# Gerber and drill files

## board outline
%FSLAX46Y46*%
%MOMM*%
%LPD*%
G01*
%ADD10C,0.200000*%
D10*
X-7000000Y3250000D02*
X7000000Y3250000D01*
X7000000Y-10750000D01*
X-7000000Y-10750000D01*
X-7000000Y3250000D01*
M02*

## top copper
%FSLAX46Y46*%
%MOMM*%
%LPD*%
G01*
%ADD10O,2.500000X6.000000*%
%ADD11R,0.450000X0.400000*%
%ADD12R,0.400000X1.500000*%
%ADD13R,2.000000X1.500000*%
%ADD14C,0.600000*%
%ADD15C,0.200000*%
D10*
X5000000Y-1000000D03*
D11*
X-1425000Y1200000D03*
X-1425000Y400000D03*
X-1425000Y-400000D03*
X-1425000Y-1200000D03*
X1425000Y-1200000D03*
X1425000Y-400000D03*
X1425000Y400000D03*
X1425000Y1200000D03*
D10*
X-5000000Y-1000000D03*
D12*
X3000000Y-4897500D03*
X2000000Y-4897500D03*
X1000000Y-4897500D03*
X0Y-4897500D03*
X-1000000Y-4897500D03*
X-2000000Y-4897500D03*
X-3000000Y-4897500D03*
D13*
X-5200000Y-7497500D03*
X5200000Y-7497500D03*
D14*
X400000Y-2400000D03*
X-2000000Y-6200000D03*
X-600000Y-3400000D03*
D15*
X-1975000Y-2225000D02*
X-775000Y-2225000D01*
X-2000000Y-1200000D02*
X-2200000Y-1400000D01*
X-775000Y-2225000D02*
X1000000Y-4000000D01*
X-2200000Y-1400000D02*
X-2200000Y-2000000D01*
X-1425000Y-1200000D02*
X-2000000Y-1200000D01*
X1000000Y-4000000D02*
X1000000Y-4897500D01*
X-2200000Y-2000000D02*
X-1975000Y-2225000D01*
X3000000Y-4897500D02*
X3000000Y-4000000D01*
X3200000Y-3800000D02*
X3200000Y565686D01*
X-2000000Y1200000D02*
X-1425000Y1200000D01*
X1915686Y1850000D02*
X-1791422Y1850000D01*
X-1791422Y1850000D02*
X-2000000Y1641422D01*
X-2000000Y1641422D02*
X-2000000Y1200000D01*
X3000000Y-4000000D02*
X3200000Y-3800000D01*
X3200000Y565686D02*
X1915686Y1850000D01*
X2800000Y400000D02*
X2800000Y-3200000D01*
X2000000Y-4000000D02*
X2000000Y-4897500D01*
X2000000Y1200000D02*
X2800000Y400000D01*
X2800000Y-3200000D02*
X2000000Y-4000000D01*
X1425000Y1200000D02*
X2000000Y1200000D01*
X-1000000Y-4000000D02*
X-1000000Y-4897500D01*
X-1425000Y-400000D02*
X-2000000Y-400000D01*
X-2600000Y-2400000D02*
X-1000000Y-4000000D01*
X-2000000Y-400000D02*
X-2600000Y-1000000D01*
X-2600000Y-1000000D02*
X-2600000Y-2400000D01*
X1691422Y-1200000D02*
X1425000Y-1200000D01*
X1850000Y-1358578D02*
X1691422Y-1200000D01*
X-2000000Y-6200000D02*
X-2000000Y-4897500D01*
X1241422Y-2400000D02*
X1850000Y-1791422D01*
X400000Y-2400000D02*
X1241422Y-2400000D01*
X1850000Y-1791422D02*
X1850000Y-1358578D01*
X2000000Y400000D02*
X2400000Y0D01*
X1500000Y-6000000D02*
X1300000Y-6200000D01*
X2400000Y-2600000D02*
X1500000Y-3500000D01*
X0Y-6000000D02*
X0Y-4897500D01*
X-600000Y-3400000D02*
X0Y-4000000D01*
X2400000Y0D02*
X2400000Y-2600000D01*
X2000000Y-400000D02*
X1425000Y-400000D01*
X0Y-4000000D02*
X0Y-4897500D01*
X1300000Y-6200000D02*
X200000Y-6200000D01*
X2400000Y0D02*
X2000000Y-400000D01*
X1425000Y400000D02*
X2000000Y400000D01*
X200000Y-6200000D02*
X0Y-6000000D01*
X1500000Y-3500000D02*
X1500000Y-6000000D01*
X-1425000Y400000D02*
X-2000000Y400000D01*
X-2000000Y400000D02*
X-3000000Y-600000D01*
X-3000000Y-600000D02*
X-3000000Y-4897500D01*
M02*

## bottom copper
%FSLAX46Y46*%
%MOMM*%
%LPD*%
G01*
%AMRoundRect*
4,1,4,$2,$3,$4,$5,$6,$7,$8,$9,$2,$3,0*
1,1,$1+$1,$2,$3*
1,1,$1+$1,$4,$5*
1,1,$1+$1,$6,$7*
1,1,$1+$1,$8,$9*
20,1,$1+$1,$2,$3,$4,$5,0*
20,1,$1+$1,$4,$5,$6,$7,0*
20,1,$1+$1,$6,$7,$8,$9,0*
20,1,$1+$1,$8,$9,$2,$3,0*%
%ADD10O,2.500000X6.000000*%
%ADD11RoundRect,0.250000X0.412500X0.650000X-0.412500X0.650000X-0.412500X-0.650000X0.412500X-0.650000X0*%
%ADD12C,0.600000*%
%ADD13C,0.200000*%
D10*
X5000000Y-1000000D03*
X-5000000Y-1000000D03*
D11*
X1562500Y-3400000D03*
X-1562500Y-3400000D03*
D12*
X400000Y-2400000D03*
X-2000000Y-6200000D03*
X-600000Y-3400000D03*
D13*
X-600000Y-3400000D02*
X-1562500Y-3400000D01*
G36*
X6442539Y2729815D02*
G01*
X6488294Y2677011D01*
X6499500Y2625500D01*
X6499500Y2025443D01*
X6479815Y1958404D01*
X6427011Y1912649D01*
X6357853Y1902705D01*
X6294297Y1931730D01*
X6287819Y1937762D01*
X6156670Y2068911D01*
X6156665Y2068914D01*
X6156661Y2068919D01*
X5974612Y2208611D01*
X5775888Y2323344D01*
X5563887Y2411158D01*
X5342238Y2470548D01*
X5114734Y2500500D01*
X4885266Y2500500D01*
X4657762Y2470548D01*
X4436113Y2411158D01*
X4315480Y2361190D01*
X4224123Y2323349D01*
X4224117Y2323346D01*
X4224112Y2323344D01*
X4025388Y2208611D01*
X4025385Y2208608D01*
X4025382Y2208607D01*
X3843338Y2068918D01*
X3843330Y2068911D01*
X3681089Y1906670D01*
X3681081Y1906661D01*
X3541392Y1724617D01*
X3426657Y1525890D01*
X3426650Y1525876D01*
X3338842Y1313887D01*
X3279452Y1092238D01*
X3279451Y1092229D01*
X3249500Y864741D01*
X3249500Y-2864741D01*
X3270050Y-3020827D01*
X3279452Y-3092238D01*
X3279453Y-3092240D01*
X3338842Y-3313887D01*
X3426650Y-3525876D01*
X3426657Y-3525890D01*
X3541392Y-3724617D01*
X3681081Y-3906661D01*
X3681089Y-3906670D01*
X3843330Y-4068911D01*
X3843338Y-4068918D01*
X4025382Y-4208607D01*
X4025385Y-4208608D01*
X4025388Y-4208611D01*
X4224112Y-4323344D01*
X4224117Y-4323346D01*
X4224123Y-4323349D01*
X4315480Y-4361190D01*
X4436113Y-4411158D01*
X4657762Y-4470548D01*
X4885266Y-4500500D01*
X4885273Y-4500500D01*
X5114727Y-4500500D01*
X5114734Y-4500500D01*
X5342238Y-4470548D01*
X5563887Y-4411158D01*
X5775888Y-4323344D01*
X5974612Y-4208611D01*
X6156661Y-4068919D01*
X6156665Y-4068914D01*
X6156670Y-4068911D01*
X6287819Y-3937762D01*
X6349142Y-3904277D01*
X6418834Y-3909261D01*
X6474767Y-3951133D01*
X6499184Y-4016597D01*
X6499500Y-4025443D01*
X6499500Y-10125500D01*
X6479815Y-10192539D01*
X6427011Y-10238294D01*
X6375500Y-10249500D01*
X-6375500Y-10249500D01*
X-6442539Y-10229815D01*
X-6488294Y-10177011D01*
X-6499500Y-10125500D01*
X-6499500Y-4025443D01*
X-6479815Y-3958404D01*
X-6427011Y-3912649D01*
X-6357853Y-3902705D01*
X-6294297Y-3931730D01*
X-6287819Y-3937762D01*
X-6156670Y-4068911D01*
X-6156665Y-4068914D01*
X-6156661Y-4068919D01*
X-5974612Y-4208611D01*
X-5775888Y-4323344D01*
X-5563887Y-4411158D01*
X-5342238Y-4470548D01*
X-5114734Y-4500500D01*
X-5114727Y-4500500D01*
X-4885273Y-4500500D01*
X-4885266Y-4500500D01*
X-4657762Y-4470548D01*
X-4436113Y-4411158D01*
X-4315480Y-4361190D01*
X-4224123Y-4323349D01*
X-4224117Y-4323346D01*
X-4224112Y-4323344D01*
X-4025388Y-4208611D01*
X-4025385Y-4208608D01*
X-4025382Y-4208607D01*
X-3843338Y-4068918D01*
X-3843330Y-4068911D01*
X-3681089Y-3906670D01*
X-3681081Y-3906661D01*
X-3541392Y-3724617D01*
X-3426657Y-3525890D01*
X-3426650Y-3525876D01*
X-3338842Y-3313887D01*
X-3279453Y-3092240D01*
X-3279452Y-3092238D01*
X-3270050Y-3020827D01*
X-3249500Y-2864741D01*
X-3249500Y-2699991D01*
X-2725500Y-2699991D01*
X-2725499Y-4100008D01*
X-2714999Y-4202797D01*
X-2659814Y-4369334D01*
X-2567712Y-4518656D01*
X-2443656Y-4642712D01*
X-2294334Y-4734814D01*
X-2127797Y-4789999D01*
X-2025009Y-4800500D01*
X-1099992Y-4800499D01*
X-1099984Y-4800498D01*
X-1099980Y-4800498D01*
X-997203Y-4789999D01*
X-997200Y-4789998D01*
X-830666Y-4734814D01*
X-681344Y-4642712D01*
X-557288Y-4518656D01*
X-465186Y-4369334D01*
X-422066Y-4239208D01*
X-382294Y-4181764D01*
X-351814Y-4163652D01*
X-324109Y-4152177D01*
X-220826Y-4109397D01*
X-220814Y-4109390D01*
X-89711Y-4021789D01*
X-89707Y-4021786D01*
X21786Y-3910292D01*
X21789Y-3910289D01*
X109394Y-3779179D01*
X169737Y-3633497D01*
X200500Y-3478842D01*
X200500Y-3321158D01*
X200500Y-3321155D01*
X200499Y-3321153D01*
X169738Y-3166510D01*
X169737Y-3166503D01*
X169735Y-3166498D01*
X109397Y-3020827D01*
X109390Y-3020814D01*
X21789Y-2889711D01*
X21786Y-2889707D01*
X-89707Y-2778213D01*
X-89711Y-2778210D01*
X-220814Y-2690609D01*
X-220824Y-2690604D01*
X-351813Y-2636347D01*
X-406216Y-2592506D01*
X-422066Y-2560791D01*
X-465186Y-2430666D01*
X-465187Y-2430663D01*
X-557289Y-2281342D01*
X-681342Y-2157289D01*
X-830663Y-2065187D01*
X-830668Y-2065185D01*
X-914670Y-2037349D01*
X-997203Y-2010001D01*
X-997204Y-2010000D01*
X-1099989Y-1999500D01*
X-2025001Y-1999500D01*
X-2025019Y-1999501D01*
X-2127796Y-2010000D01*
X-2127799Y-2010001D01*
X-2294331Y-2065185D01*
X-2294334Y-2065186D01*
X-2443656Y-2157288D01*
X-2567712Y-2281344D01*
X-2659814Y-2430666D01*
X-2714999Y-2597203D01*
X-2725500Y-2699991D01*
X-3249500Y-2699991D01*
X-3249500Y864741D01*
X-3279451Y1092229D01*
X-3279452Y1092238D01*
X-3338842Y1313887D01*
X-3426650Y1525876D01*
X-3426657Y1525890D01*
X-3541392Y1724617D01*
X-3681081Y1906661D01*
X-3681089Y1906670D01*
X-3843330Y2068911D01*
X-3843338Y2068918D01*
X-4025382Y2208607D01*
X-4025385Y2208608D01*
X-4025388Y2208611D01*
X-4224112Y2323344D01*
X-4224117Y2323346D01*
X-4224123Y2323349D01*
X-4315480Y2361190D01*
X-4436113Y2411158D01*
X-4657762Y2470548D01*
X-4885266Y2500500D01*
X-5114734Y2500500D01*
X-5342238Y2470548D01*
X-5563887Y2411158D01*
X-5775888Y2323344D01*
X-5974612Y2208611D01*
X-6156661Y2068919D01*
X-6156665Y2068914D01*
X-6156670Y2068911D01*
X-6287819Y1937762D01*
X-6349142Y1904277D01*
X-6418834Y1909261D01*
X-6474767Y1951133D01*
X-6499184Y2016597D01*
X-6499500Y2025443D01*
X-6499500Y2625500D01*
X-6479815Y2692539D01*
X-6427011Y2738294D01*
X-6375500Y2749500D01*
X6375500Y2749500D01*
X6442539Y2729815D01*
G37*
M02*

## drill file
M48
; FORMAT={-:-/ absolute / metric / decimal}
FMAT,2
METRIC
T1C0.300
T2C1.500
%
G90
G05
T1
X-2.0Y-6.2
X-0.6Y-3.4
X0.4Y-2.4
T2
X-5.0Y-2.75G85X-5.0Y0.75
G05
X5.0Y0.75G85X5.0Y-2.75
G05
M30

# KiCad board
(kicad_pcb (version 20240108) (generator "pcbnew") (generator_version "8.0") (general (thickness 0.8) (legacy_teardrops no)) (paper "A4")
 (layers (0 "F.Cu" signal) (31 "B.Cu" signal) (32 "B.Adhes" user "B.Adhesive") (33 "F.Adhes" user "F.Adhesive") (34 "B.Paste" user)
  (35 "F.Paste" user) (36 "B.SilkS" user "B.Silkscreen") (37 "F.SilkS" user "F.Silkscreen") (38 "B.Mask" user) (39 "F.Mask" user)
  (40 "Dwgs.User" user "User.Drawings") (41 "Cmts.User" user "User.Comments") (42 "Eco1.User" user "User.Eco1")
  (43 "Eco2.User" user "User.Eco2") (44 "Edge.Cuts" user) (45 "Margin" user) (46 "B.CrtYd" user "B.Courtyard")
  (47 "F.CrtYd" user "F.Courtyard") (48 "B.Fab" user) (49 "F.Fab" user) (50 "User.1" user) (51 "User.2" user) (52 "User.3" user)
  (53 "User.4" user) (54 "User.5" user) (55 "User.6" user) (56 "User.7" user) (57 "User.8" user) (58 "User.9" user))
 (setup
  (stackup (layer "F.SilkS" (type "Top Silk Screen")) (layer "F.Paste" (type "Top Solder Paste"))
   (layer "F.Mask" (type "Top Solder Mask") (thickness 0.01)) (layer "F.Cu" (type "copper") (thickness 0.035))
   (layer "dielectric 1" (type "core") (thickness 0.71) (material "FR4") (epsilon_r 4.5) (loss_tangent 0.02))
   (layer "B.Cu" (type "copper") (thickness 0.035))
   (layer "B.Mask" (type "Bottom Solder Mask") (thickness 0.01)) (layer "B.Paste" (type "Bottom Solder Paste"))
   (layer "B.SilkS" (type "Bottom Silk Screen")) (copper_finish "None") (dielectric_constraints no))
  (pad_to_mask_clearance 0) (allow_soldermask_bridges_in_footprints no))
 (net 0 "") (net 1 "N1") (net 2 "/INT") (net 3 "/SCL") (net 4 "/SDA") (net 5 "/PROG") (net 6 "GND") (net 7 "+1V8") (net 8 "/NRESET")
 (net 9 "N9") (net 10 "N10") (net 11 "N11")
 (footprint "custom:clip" (layer "F.Cu") (at 5 1 -90)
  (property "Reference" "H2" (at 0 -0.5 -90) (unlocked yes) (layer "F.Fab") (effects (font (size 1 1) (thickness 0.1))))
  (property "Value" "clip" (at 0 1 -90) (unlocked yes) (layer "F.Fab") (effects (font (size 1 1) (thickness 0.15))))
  (pad "1" thru_hole oval (at 0 0 270) (size 6 2.5) (drill oval 5 1.5) (layers "*.Cu" "*.Mask") (remove_unused_layers no) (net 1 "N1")
   (thermal_bridge_angle 45)))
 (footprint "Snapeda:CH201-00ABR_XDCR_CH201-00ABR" (layer "F.Cu") (at 0 0)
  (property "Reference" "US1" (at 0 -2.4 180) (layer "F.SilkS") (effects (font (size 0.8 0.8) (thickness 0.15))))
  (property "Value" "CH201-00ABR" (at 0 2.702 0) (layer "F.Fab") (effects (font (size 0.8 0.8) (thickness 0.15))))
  (pad "1" smd rect (at -1.425 -1.2) (size 0.45 0.4) (layers "F.Cu") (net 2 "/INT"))
  (pad "2" smd rect (at -1.425 -0.4) (size 0.45 0.4) (layers "F.Cu") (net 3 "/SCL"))
  (pad "3" smd rect (at -1.425 0.4) (size 0.45 0.4) (layers "F.Cu") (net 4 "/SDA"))
  (pad "4" smd rect (at -1.425 1.2) (size 0.45 0.4) (layers "F.Cu") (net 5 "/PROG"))
  (pad "5" smd rect (at 1.425 1.2) (size 0.45 0.4) (layers "F.Cu") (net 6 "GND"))
  (pad "6" smd rect (at 1.425 0.4) (size 0.45 0.4) (layers "F.Cu") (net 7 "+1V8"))
  (pad "7" smd rect (at 1.425 -0.4) (size 0.45 0.4) (layers "F.Cu") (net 7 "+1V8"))
  (pad "8" smd rect (at 1.425 -1.2) (size 0.45 0.4) (layers "F.Cu") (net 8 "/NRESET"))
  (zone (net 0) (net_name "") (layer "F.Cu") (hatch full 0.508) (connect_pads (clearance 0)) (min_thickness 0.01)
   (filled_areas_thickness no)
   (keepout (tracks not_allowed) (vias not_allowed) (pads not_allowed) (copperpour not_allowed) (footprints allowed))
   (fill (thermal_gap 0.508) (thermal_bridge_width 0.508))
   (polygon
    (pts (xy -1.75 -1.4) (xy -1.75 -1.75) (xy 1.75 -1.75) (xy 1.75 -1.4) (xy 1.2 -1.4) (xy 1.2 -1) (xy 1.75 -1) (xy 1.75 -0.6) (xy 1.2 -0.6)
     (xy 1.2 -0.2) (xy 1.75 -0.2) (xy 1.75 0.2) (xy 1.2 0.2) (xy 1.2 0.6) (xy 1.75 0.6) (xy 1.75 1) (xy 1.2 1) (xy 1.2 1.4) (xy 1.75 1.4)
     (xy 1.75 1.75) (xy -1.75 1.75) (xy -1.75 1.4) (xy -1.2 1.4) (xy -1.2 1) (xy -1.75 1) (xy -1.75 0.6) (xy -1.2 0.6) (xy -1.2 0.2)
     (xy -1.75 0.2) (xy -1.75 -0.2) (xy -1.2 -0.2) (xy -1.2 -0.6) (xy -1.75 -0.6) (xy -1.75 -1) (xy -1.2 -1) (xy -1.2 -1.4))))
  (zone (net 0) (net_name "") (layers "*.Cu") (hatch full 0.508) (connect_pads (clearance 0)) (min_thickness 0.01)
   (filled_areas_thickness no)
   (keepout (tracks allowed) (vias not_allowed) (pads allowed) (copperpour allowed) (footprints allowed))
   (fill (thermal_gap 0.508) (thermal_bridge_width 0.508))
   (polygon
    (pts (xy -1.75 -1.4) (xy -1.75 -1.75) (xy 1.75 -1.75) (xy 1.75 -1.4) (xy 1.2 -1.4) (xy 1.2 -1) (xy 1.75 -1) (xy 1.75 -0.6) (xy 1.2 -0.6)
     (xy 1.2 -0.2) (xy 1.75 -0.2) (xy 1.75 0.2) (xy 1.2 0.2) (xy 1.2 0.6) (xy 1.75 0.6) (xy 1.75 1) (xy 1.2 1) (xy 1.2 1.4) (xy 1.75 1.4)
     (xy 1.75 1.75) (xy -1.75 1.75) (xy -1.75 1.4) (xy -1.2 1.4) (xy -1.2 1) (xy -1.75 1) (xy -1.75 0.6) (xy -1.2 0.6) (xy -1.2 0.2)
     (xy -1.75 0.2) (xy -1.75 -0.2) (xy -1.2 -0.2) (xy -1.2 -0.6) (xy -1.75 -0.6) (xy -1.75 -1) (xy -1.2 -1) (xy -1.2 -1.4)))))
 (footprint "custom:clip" (layer "F.Cu") (at -5 1 90)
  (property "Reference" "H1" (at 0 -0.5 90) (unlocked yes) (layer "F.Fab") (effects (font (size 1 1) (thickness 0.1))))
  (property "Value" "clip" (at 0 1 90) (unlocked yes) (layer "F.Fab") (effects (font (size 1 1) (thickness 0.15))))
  (pad "1" thru_hole oval (at 0 0 90) (size 6 2.5) (drill oval 5 1.5) (layers "*.Cu" "*.Mask") (remove_unused_layers no) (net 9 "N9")
   (thermal_bridge_angle 45)))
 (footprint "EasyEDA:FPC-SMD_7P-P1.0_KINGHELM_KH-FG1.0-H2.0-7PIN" (layer "F.Cu") (at 0 6.1975)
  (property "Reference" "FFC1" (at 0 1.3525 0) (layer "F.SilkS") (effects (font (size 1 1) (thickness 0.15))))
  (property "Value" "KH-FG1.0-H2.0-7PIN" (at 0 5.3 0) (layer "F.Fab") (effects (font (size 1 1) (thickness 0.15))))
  (pad "1" smd rect (at 3 -1.3 180) (size 0.4 1.5) (layers "F.Cu" "F.Paste" "F.Mask") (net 2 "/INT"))
  (pad "2" smd rect (at 2 -1.3 180) (size 0.4 1.5) (layers "F.Cu" "F.Paste" "F.Mask") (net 8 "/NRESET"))
  (pad "3" smd rect (at 1 -1.3 180) (size 0.4 1.5) (layers "F.Cu" "F.Paste" "F.Mask") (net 5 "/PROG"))
  (pad "4" smd rect (at 0 -1.3 180) (size 0.4 1.5) (layers "F.Cu" "F.Paste" "F.Mask") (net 7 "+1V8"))
  (pad "5" smd rect (at -1 -1.3 180) (size 0.4 1.5) (layers "F.Cu" "F.Paste" "F.Mask") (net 4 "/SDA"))
  (pad "6" smd rect (at -2 -1.3 180) (size 0.4 1.5) (layers "F.Cu" "F.Paste" "F.Mask") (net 6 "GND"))
  (pad "7" smd rect (at -3 -1.3 180) (size 0.4 1.5) (layers "F.Cu" "F.Paste" "F.Mask") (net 3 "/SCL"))
  (pad "8" smd rect (at -5.2 1.3 180) (size 2 1.5) (layers "F.Cu" "F.Paste" "F.Mask") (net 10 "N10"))
  (pad "9" smd rect (at 5.2 1.3 180) (size 2 1.5) (layers "F.Cu" "F.Paste" "F.Mask") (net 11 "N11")))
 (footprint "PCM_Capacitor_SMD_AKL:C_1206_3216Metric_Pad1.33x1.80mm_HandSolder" (layer "B.Cu") (at 0 3.4 180)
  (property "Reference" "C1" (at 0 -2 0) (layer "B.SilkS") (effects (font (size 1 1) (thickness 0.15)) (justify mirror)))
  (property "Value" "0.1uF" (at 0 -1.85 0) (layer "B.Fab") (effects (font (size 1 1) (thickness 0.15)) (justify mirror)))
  (pad "1" smd roundrect (at -1.5625 0 180) (size 1.325 1.8) (layers "B.Cu" "B.Paste" "B.Mask") (roundrect_rratio 0.188679) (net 6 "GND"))
  (pad "2" smd roundrect (at 1.5625 0 180) (size 1.325 1.8) (layers "B.Cu" "B.Paste" "B.Mask") (roundrect_rratio 0.188679) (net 7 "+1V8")))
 (gr_rect (start -7 -3.25) (end 7 10.75) (stroke (width 0.2) (type default)) (fill none) (layer "Edge.Cuts"))
 (segment (start -1.975 2.225) (end -0.775 2.225) (width 0.2) (layer "F.Cu") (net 5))
 (segment (start -2 1.2) (end -2.2 1.4) (width 0.2) (layer "F.Cu") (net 5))
 (segment (start -0.775 2.225) (end 1 4) (width 0.2) (layer "F.Cu") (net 5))
 (segment (start -2.2 1.4) (end -2.2 2) (width 0.2) (layer "F.Cu") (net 5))
 (segment (start -1.425 1.2) (end -2 1.2) (width 0.2) (layer "F.Cu") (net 5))
 (segment (start 1 4) (end 1 4.8975) (width 0.2) (layer "F.Cu") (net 5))
 (segment (start -2.2 2) (end -1.975 2.225) (width 0.2) (layer "F.Cu") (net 5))
 (segment (start 3 4.8975) (end 3 4) (width 0.2) (layer "F.Cu") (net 2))
 (segment (start 3.2 3.8) (end 3.2 -0.565686) (width 0.2) (layer "F.Cu") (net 2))
 (segment (start -2 -1.2) (end -1.425 -1.2) (width 0.2) (layer "F.Cu") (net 2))
 (segment (start 1.915686 -1.85) (end -1.791422 -1.85) (width 0.2) (layer "F.Cu") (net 2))
 (segment (start -1.791422 -1.85) (end -2 -1.641422) (width 0.2) (layer "F.Cu") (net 2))
 (segment (start -2 -1.641422) (end -2 -1.2) (width 0.2) (layer "F.Cu") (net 2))
 (segment (start 3 4) (end 3.2 3.8) (width 0.2) (layer "F.Cu") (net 2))
 (segment (start 3.2 -0.565686) (end 1.915686 -1.85) (width 0.2) (layer "F.Cu") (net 2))
 (segment (start 2.8 -0.4) (end 2.8 3.2) (width 0.2) (layer "F.Cu") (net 8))
 (segment (start 2 4) (end 2 4.8975) (width 0.2) (layer "F.Cu") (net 8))
 (segment (start 2 -1.2) (end 2.8 -0.4) (width 0.2) (layer "F.Cu") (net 8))
 (segment (start 2.8 3.2) (end 2 4) (width 0.2) (layer "F.Cu") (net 8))
 (segment (start 1.425 -1.2) (end 2 -1.2) (width 0.2) (layer "F.Cu") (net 8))
 (segment (start -1 4) (end -1 4.8975) (width 0.2) (layer "F.Cu") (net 4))
 (segment (start -1.425 0.4) (end -2 0.4) (width 0.2) (layer "F.Cu") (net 4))
 (segment (start -2.6 2.4) (end -1 4) (width 0.2) (layer "F.Cu") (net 4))
 (segment (start -2 0.4) (end -2.6 1) (width 0.2) (layer "F.Cu") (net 4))
 (segment (start -2.6 1) (end -2.6 2.4) (width 0.2) (layer "F.Cu") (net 4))
 (segment (start 1.691422 1.2) (end 1.425 1.2) (width 0.2) (layer "F.Cu") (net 6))
 (segment (start 1.85 1.358578) (end 1.691422 1.2) (width 0.2) (layer "F.Cu") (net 6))
 (segment (start -2 6.2) (end -2 4.8975) (width 0.2) (layer "F.Cu") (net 6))
 (segment (start 1.241422 2.4) (end 1.85 1.791422) (width 0.2) (layer "F.Cu") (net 6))
 (segment (start 0.4 2.4) (end 1.241422 2.4) (width 0.2) (layer "F.Cu") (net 6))
 (segment (start 1.85 1.791422) (end 1.85 1.358578) (width 0.2) (layer "F.Cu") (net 6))
 (via (at 0.4 2.4) (size 0.6) (drill 0.3) (layers "F.Cu" "B.Cu") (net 6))
 (via (at -2 6.2) (size 0.6) (drill 0.3) (layers "F.Cu" "B.Cu") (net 6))
 (segment (start 2 -0.4) (end 2.4 0) (width 0.2) (layer "F.Cu") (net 7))
 (segment (start 1.5 6) (end 1.3 6.2) (width 0.2) (layer "F.Cu") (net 7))
 (segment (start 2.4 2.6) (end 1.5 3.5) (width 0.2) (layer "F.Cu") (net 7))
 (segment (start 0 6) (end 0 4.8975) (width 0.2) (layer "F.Cu") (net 7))
 (segment (start -0.6 3.4) (end 0 4) (width 0.2) (layer "F.Cu") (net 7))
 (segment (start 2.4 0) (end 2.4 2.6) (width 0.2) (layer "F.Cu") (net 7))
 (segment (start 2 0.4) (end 1.425 0.4) (width 0.2) (layer "F.Cu") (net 7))
 (segment (start 0 4) (end 0 4.8975) (width 0.2) (layer "F.Cu") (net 7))
 (segment (start 1.3 6.2) (end 0.2 6.2) (width 0.2) (layer "F.Cu") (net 7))
 (segment (start 2.4 0) (end 2 0.4) (width 0.2) (layer "F.Cu") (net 7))
 (segment (start 1.425 -0.4) (end 2 -0.4) (width 0.2) (layer "F.Cu") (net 7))
 (segment (start 0.2 6.2) (end 0 6) (width 0.2) (layer "F.Cu") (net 7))
 (segment (start 1.5 3.5) (end 1.5 6) (width 0.2) (layer "F.Cu") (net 7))
 (via (at -0.6 3.4) (size 0.6) (drill 0.3) (layers "F.Cu" "B.Cu") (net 7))
 (segment (start -0.6 3.4) (end -1.5625 3.4) (width 0.2) (layer "B.Cu") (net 7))
 (segment (start -1.425 -0.4) (end -2 -0.4) (width 0.2) (layer "F.Cu") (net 3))
 (segment (start -2 -0.4) (end -3 0.6) (width 0.2) (layer "F.Cu") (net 3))
 (segment (start -3 0.6) (end -3 4.8975) (width 0.2) (layer "F.Cu") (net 3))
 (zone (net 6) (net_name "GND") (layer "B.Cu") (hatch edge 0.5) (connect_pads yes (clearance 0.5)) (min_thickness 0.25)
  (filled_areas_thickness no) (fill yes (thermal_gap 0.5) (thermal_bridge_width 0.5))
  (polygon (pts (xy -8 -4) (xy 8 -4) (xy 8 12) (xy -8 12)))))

